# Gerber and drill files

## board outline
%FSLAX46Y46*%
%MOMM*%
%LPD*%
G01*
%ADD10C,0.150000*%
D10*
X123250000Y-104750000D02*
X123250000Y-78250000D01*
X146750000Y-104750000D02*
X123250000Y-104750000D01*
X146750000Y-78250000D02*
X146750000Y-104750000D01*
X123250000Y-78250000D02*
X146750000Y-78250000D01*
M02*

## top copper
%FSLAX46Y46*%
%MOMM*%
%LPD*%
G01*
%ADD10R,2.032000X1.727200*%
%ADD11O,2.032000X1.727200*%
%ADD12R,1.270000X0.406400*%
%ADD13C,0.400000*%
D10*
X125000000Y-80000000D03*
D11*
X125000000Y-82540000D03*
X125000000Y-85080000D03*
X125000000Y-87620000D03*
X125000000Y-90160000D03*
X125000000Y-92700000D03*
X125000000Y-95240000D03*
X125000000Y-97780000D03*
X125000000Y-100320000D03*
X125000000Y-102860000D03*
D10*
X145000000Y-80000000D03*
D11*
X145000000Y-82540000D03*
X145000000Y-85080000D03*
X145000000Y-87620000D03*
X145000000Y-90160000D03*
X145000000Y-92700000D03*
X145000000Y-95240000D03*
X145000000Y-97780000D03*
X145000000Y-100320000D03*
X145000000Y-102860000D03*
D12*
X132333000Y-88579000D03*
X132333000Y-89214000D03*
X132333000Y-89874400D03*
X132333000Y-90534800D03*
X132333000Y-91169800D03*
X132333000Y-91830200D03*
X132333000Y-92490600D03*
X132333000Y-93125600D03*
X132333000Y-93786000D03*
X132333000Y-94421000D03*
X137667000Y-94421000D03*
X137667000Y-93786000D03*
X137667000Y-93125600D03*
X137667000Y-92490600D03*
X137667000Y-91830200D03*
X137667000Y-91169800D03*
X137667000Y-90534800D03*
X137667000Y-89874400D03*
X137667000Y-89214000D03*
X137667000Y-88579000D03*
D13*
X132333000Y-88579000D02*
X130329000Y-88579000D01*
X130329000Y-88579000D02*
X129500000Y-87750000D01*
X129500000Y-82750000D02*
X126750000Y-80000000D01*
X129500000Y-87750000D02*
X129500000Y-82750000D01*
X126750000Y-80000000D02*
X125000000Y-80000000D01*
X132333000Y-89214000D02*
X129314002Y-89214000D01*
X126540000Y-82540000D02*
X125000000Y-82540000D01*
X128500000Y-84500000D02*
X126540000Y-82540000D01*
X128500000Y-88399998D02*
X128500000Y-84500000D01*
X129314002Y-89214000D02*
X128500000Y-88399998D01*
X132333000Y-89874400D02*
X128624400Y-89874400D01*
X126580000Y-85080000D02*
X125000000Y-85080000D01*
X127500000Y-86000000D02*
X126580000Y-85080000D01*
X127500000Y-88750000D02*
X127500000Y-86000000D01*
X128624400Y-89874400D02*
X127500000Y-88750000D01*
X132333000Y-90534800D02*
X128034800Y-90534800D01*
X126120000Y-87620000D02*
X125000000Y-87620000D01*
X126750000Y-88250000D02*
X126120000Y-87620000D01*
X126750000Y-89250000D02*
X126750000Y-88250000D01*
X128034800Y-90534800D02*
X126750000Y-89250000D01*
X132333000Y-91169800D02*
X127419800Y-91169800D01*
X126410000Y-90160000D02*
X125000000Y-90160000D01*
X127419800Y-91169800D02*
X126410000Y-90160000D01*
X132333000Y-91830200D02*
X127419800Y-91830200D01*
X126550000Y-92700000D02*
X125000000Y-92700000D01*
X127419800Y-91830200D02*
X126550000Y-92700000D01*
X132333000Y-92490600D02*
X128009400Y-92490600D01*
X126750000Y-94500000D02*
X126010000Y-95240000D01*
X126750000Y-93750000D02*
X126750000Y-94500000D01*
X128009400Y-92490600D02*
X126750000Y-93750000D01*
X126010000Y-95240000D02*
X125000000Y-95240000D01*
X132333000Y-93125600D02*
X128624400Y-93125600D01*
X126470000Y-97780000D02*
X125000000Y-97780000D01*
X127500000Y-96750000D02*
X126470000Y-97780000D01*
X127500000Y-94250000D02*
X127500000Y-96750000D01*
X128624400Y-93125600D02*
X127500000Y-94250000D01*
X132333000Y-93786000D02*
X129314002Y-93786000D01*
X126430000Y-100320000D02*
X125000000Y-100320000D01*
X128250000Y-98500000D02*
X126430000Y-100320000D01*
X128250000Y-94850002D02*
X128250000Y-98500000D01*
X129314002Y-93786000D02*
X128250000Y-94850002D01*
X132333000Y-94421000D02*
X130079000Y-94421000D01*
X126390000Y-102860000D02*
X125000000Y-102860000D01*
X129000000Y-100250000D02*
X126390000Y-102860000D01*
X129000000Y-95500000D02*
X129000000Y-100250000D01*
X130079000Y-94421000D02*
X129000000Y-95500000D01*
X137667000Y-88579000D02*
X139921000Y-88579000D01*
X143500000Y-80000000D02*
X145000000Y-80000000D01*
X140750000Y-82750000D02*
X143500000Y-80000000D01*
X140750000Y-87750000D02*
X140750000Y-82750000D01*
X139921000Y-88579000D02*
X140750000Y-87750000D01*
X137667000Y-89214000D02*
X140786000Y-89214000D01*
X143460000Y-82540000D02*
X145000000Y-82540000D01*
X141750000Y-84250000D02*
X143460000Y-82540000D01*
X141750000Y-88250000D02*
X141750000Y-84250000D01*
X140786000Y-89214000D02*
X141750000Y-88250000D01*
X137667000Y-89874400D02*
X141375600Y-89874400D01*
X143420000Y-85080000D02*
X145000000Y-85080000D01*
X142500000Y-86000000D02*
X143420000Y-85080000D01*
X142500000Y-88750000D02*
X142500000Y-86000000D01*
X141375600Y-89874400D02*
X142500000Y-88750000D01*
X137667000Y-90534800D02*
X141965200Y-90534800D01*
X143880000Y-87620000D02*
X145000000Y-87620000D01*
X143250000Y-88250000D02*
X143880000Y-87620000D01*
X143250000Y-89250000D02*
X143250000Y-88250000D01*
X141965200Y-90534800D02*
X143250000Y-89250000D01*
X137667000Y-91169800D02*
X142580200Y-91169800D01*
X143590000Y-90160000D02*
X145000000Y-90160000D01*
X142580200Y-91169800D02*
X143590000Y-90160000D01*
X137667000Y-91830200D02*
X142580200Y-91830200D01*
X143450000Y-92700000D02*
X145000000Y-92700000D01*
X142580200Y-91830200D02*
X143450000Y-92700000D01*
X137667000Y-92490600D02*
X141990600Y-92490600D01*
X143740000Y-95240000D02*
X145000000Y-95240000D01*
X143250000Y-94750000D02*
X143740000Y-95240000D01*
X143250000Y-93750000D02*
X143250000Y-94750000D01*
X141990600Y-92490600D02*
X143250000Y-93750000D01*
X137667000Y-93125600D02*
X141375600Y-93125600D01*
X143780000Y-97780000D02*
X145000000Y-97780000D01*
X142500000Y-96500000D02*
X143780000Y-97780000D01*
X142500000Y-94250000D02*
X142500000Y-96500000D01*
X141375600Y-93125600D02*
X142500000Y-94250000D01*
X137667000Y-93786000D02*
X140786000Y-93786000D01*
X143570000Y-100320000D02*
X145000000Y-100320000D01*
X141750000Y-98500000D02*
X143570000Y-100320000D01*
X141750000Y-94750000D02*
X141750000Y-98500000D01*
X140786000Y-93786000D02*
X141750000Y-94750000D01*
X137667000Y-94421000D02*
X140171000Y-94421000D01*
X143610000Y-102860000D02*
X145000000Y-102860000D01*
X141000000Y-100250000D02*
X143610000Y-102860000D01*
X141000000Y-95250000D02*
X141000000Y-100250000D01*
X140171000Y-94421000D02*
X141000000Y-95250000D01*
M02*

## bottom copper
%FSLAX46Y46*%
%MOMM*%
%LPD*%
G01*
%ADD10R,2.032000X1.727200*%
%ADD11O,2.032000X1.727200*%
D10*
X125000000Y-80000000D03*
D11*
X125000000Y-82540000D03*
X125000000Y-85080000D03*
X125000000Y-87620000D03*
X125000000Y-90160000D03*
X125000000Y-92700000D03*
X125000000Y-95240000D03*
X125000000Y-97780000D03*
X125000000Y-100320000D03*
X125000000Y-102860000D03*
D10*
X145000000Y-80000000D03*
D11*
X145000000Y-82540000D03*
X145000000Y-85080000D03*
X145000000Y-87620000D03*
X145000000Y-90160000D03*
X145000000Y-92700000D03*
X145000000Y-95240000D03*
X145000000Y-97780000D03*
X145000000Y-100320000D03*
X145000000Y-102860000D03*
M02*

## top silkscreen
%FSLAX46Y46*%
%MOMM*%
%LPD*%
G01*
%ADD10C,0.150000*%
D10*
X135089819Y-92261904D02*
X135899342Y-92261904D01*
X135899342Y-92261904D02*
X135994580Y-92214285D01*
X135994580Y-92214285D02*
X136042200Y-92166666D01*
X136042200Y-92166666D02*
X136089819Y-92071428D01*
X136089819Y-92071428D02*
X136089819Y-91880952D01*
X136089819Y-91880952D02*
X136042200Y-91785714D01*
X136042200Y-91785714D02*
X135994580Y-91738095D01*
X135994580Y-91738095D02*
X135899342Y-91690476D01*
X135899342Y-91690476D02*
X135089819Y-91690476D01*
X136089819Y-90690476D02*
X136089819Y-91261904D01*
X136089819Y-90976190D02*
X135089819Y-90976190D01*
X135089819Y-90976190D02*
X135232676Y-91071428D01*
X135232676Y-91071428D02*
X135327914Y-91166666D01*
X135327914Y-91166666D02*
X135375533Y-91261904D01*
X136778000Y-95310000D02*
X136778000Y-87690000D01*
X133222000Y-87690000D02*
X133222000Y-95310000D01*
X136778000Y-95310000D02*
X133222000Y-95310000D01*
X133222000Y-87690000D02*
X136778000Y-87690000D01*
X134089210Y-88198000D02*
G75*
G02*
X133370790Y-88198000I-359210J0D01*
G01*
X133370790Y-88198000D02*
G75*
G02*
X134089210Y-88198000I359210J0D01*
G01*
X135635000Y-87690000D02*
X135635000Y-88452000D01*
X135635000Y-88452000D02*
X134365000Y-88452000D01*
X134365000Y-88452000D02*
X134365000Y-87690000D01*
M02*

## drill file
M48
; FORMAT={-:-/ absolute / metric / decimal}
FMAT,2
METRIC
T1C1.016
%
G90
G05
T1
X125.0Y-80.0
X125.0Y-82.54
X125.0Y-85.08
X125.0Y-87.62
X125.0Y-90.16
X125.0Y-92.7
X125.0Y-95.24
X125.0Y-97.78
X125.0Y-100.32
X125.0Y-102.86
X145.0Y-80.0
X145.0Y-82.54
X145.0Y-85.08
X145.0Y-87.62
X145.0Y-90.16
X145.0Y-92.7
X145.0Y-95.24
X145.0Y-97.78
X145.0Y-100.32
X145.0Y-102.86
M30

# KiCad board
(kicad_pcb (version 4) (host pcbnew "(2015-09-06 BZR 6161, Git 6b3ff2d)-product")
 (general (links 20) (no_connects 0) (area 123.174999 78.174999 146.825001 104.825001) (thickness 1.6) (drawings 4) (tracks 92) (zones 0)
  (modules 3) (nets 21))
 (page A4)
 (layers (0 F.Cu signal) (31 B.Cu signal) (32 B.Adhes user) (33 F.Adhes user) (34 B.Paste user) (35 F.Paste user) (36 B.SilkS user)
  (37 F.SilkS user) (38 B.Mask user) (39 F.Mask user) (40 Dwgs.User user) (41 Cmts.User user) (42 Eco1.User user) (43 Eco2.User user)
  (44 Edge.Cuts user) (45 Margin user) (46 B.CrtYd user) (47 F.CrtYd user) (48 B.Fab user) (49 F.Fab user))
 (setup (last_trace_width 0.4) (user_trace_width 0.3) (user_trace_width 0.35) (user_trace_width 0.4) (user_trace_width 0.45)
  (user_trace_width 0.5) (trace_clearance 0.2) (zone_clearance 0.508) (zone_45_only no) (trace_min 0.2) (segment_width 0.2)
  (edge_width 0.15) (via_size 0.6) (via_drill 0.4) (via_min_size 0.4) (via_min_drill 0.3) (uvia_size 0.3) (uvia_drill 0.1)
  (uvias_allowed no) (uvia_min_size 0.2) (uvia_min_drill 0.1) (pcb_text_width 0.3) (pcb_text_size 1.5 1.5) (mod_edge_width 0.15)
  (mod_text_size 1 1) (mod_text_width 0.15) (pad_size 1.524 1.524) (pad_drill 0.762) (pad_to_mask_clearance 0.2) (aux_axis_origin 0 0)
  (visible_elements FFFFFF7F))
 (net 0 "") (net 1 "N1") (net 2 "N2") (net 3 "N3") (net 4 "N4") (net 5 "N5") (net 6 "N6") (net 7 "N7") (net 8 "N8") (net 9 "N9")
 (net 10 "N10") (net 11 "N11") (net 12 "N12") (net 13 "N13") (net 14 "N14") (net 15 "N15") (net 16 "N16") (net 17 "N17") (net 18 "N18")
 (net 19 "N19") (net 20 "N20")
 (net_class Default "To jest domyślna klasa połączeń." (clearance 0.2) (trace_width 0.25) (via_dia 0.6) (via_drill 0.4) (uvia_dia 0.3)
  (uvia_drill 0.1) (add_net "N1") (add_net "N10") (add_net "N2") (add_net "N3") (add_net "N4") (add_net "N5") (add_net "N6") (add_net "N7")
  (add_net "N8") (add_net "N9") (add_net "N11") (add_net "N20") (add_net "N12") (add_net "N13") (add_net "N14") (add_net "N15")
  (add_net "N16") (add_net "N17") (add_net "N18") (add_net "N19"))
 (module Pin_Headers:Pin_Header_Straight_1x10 (layer B.Cu) (at 125 80 180)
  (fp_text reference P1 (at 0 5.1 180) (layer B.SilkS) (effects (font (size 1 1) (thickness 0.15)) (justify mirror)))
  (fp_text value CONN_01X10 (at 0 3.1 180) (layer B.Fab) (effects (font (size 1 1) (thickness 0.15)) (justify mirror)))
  (pad 1 thru_hole rect (at 0 0 180) (size 2.032 1.7272) (drill 1.016) (layers *.Cu *.Mask B.SilkS) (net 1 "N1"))
  (pad 2 thru_hole oval (at 0 -2.54 180) (size 2.032 1.7272) (drill 1.016) (layers *.Cu *.Mask B.SilkS) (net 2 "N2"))
  (pad 3 thru_hole oval (at 0 -5.08 180) (size 2.032 1.7272) (drill 1.016) (layers *.Cu *.Mask B.SilkS) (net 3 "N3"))
  (pad 4 thru_hole oval (at 0 -7.62 180) (size 2.032 1.7272) (drill 1.016) (layers *.Cu *.Mask B.SilkS) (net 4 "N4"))
  (pad 5 thru_hole oval (at 0 -10.16 180) (size 2.032 1.7272) (drill 1.016) (layers *.Cu *.Mask B.SilkS) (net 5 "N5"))
  (pad 6 thru_hole oval (at 0 -12.7 180) (size 2.032 1.7272) (drill 1.016) (layers *.Cu *.Mask B.SilkS) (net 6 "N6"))
  (pad 7 thru_hole oval (at 0 -15.24 180) (size 2.032 1.7272) (drill 1.016) (layers *.Cu *.Mask B.SilkS) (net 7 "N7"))
  (pad 8 thru_hole oval (at 0 -17.78 180) (size 2.032 1.7272) (drill 1.016) (layers *.Cu *.Mask B.SilkS) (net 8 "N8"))
  (pad 9 thru_hole oval (at 0 -20.32 180) (size 2.032 1.7272) (drill 1.016) (layers *.Cu *.Mask B.SilkS) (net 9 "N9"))
  (pad 10 thru_hole oval (at 0 -22.86 180) (size 2.032 1.7272) (drill 1.016) (layers *.Cu *.Mask B.SilkS) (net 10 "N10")))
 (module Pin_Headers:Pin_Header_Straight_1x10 (layer B.Cu) (at 145 80 180)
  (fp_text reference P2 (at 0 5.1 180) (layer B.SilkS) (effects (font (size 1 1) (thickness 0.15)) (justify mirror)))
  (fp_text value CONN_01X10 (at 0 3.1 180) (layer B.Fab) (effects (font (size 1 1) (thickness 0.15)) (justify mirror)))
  (pad 1 thru_hole rect (at 0 0 180) (size 2.032 1.7272) (drill 1.016) (layers *.Cu *.Mask B.SilkS) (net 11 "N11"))
  (pad 2 thru_hole oval (at 0 -2.54 180) (size 2.032 1.7272) (drill 1.016) (layers *.Cu *.Mask B.SilkS) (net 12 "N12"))
  (pad 3 thru_hole oval (at 0 -5.08 180) (size 2.032 1.7272) (drill 1.016) (layers *.Cu *.Mask B.SilkS) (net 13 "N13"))
  (pad 4 thru_hole oval (at 0 -7.62 180) (size 2.032 1.7272) (drill 1.016) (layers *.Cu *.Mask B.SilkS) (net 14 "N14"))
  (pad 5 thru_hole oval (at 0 -10.16 180) (size 2.032 1.7272) (drill 1.016) (layers *.Cu *.Mask B.SilkS) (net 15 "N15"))
  (pad 6 thru_hole oval (at 0 -12.7 180) (size 2.032 1.7272) (drill 1.016) (layers *.Cu *.Mask B.SilkS) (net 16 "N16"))
  (pad 7 thru_hole oval (at 0 -15.24 180) (size 2.032 1.7272) (drill 1.016) (layers *.Cu *.Mask B.SilkS) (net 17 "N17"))
  (pad 8 thru_hole oval (at 0 -17.78 180) (size 2.032 1.7272) (drill 1.016) (layers *.Cu *.Mask B.SilkS) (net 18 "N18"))
  (pad 9 thru_hole oval (at 0 -20.32 180) (size 2.032 1.7272) (drill 1.016) (layers *.Cu *.Mask B.SilkS) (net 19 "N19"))
  (pad 10 thru_hole oval (at 0 -22.86 180) (size 2.032 1.7272) (drill 1.016) (layers *.Cu *.Mask B.SilkS) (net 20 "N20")))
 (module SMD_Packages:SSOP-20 (layer F.Cu) (at 135 91.5 270)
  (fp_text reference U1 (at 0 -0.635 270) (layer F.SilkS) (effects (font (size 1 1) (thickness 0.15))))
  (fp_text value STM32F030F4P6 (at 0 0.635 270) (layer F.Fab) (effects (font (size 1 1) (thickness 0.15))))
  (fp_line (start 3.81 -1.778) (end -3.81 -1.778) (layer F.SilkS) (width 0.15))
  (fp_line (start -3.81 1.778) (end 3.81 1.778) (layer F.SilkS) (width 0.15))
  (fp_line (start 3.81 -1.778) (end 3.81 1.778) (layer F.SilkS) (width 0.15))
  (fp_line (start -3.81 1.778) (end -3.81 -1.778) (layer F.SilkS) (width 0.15))
  (fp_circle (center -3.302 1.27) (end -3.556 1.016) (layer F.SilkS) (width 0.15))
  (fp_line (start -3.81 -0.635) (end -3.048 -0.635) (layer F.SilkS) (width 0.15))
  (fp_line (start -3.048 -0.635) (end -3.048 0.635) (layer F.SilkS) (width 0.15))
  (fp_line (start -3.048 0.635) (end -3.81 0.635) (layer F.SilkS) (width 0.15))
  (pad 1 smd rect (at -2.921 2.667 270) (size 0.4064 1.27) (layers F.Cu F.Paste F.Mask) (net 1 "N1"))
  (pad 2 smd rect (at -2.286 2.667 270) (size 0.4064 1.27) (layers F.Cu F.Paste F.Mask) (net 2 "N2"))
  (pad 3 smd rect (at -1.6256 2.667 270) (size 0.4064 1.27) (layers F.Cu F.Paste F.Mask) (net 3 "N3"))
  (pad 4 smd rect (at -0.9652 2.667 270) (size 0.4064 1.27) (layers F.Cu F.Paste F.Mask) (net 4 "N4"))
  (pad 5 smd rect (at -0.3302 2.667 270) (size 0.4064 1.27) (layers F.Cu F.Paste F.Mask) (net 5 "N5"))
  (pad 6 smd rect (at 0.3302 2.667 270) (size 0.4064 1.27) (layers F.Cu F.Paste F.Mask) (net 6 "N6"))
  (pad 7 smd rect (at 0.9906 2.667 270) (size 0.4064 1.27) (layers F.Cu F.Paste F.Mask) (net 7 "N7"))
  (pad 8 smd rect (at 1.6256 2.667 270) (size 0.4064 1.27) (layers F.Cu F.Paste F.Mask) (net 8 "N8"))
  (pad 9 smd rect (at 2.286 2.667 270) (size 0.4064 1.27) (layers F.Cu F.Paste F.Mask) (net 9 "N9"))
  (pad 10 smd rect (at 2.921 2.667 270) (size 0.4064 1.27) (layers F.Cu F.Paste F.Mask) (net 10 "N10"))
  (pad 11 smd rect (at 2.921 -2.667 270) (size 0.4064 1.27) (layers F.Cu F.Paste F.Mask) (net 20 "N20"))
  (pad 12 smd rect (at 2.286 -2.667 270) (size 0.4064 1.27) (layers F.Cu F.Paste F.Mask) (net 19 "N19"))
  (pad 13 smd rect (at 1.6256 -2.667 270) (size 0.4064 1.27) (layers F.Cu F.Paste F.Mask) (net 18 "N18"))
  (pad 14 smd rect (at 0.9906 -2.667 270) (size 0.4064 1.27) (layers F.Cu F.Paste F.Mask) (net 17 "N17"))
  (pad 15 smd rect (at 0.3302 -2.667 270) (size 0.4064 1.27) (layers F.Cu F.Paste F.Mask) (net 16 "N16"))
  (pad 16 smd rect (at -0.3302 -2.667 270) (size 0.4064 1.27) (layers F.Cu F.Paste F.Mask) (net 15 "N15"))
  (pad 17 smd rect (at -0.9652 -2.667 270) (size 0.4064 1.27) (layers F.Cu F.Paste F.Mask) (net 14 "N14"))
  (pad 18 smd rect (at -1.6256 -2.667 270) (size 0.4064 1.27) (layers F.Cu F.Paste F.Mask) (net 13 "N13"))
  (pad 19 smd rect (at -2.286 -2.667 270) (size 0.4064 1.27) (layers F.Cu F.Paste F.Mask) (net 12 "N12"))
  (pad 20 smd rect (at -2.921 -2.667 270) (size 0.4064 1.27) (layers F.Cu F.Paste F.Mask) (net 11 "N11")))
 (gr_line (start 123.25 104.75) (end 123.25 78.25) (angle 90) (layer Edge.Cuts) (width 0.15))
 (gr_line (start 146.75 104.75) (end 123.25 104.75) (angle 90) (layer Edge.Cuts) (width 0.15))
 (gr_line (start 146.75 78.25) (end 146.75 104.75) (angle 90) (layer Edge.Cuts) (width 0.15))
 (gr_line (start 123.25 78.25) (end 146.75 78.25) (angle 90) (layer Edge.Cuts) (width 0.15))
 (segment (start 132.333 88.579) (end 130.329 88.579) (width 0.4) (layer F.Cu) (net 1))
 (segment (start 130.329 88.579) (end 129.5 87.75) (width 0.4) (layer F.Cu) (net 1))
 (segment (start 129.5 82.75) (end 126.75 80) (width 0.4) (layer F.Cu) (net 1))
 (segment (start 129.5 87.75) (end 129.5 82.75) (width 0.4) (layer F.Cu) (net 1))
 (segment (start 126.75 80) (end 125 80) (width 0.4) (layer F.Cu) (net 1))
 (segment (start 132.333 89.214) (end 129.314002 89.214) (width 0.4) (layer F.Cu) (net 2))
 (segment (start 126.54 82.54) (end 125 82.54) (width 0.4) (layer F.Cu) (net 2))
 (segment (start 128.5 84.5) (end 126.54 82.54) (width 0.4) (layer F.Cu) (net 2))
 (segment (start 128.5 88.399998) (end 128.5 84.5) (width 0.4) (layer F.Cu) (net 2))
 (segment (start 129.314002 89.214) (end 128.5 88.399998) (width 0.4) (layer F.Cu) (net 2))
 (segment (start 132.333 89.8744) (end 128.6244 89.8744) (width 0.4) (layer F.Cu) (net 3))
 (segment (start 126.58 85.08) (end 125 85.08) (width 0.4) (layer F.Cu) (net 3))
 (segment (start 127.5 86) (end 126.58 85.08) (width 0.4) (layer F.Cu) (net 3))
 (segment (start 127.5 88.75) (end 127.5 86) (width 0.4) (layer F.Cu) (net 3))
 (segment (start 128.6244 89.8744) (end 127.5 88.75) (width 0.4) (layer F.Cu) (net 3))
 (segment (start 132.333 90.5348) (end 128.0348 90.5348) (width 0.4) (layer F.Cu) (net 4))
 (segment (start 126.12 87.62) (end 125 87.62) (width 0.4) (layer F.Cu) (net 4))
 (segment (start 126.75 88.25) (end 126.12 87.62) (width 0.4) (layer F.Cu) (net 4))
 (segment (start 126.75 89.25) (end 126.75 88.25) (width 0.4) (layer F.Cu) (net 4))
 (segment (start 128.0348 90.5348) (end 126.75 89.25) (width 0.4) (layer F.Cu) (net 4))
 (segment (start 132.333 91.1698) (end 127.4198 91.1698) (width 0.4) (layer F.Cu) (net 5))
 (segment (start 126.41 90.16) (end 125 90.16) (width 0.4) (layer F.Cu) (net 5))
 (segment (start 127.4198 91.1698) (end 126.41 90.16) (width 0.4) (layer F.Cu) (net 5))
 (segment (start 132.333 91.8302) (end 127.4198 91.8302) (width 0.4) (layer F.Cu) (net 6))
 (segment (start 126.55 92.7) (end 125 92.7) (width 0.4) (layer F.Cu) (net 6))
 (segment (start 127.4198 91.8302) (end 126.55 92.7) (width 0.4) (layer F.Cu) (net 6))
 (segment (start 132.333 92.4906) (end 128.0094 92.4906) (width 0.4) (layer F.Cu) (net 7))
 (segment (start 126.75 94.5) (end 126.01 95.24) (width 0.4) (layer F.Cu) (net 7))
 (segment (start 126.75 93.75) (end 126.75 94.5) (width 0.4) (layer F.Cu) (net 7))
 (segment (start 128.0094 92.4906) (end 126.75 93.75) (width 0.4) (layer F.Cu) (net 7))
 (segment (start 126.01 95.24) (end 125 95.24) (width 0.4) (layer F.Cu) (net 7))
 (segment (start 132.333 93.1256) (end 128.6244 93.1256) (width 0.4) (layer F.Cu) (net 8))
 (segment (start 126.47 97.78) (end 125 97.78) (width 0.4) (layer F.Cu) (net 8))
 (segment (start 127.5 96.75) (end 126.47 97.78) (width 0.4) (layer F.Cu) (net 8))
 (segment (start 127.5 94.25) (end 127.5 96.75) (width 0.4) (layer F.Cu) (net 8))
 (segment (start 128.6244 93.1256) (end 127.5 94.25) (width 0.4) (layer F.Cu) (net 8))
 (segment (start 132.333 93.786) (end 129.314002 93.786) (width 0.4) (layer F.Cu) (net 9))
 (segment (start 126.43 100.32) (end 125 100.32) (width 0.4) (layer F.Cu) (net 9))
 (segment (start 128.25 98.5) (end 126.43 100.32) (width 0.4) (layer F.Cu) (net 9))
 (segment (start 128.25 94.850002) (end 128.25 98.5) (width 0.4) (layer F.Cu) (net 9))
 (segment (start 129.314002 93.786) (end 128.25 94.850002) (width 0.4) (layer F.Cu) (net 9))
 (segment (start 132.333 94.421) (end 130.079 94.421) (width 0.4) (layer F.Cu) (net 10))
 (segment (start 126.39 102.86) (end 125 102.86) (width 0.4) (layer F.Cu) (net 10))
 (segment (start 129 100.25) (end 126.39 102.86) (width 0.4) (layer F.Cu) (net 10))
 (segment (start 129 95.5) (end 129 100.25) (width 0.4) (layer F.Cu) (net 10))
 (segment (start 130.079 94.421) (end 129 95.5) (width 0.4) (layer F.Cu) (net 10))
 (segment (start 137.667 88.579) (end 139.921 88.579) (width 0.4) (layer F.Cu) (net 11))
 (segment (start 143.5 80) (end 145 80) (width 0.4) (layer F.Cu) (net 11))
 (segment (start 140.75 82.75) (end 143.5 80) (width 0.4) (layer F.Cu) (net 11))
 (segment (start 140.75 87.75) (end 140.75 82.75) (width 0.4) (layer F.Cu) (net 11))
 (segment (start 139.921 88.579) (end 140.75 87.75) (width 0.4) (layer F.Cu) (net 11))
 (segment (start 137.667 89.214) (end 140.786 89.214) (width 0.4) (layer F.Cu) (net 12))
 (segment (start 143.46 82.54) (end 145 82.54) (width 0.4) (layer F.Cu) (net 12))
 (segment (start 141.75 84.25) (end 143.46 82.54) (width 0.4) (layer F.Cu) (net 12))
 (segment (start 141.75 88.25) (end 141.75 84.25) (width 0.4) (layer F.Cu) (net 12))
 (segment (start 140.786 89.214) (end 141.75 88.25) (width 0.4) (layer F.Cu) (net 12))
 (segment (start 137.667 89.8744) (end 141.3756 89.8744) (width 0.4) (layer F.Cu) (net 13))
 (segment (start 143.42 85.08) (end 145 85.08) (width 0.4) (layer F.Cu) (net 13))
 (segment (start 142.5 86) (end 143.42 85.08) (width 0.4) (layer F.Cu) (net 13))
 (segment (start 142.5 88.75) (end 142.5 86) (width 0.4) (layer F.Cu) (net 13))
 (segment (start 141.3756 89.8744) (end 142.5 88.75) (width 0.4) (layer F.Cu) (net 13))
 (segment (start 137.667 90.5348) (end 141.9652 90.5348) (width 0.4) (layer F.Cu) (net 14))
 (segment (start 143.88 87.62) (end 145 87.62) (width 0.4) (layer F.Cu) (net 14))
 (segment (start 143.25 88.25) (end 143.88 87.62) (width 0.4) (layer F.Cu) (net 14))
 (segment (start 143.25 89.25) (end 143.25 88.25) (width 0.4) (layer F.Cu) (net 14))
 (segment (start 141.9652 90.5348) (end 143.25 89.25) (width 0.4) (layer F.Cu) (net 14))
 (segment (start 137.667 91.1698) (end 142.5802 91.1698) (width 0.4) (layer F.Cu) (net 15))
 (segment (start 143.59 90.16) (end 145 90.16) (width 0.4) (layer F.Cu) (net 15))
 (segment (start 142.5802 91.1698) (end 143.59 90.16) (width 0.4) (layer F.Cu) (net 15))
 (segment (start 137.667 91.8302) (end 142.5802 91.8302) (width 0.4) (layer F.Cu) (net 16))
 (segment (start 143.45 92.7) (end 145 92.7) (width 0.4) (layer F.Cu) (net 16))
 (segment (start 142.5802 91.8302) (end 143.45 92.7) (width 0.4) (layer F.Cu) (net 16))
 (segment (start 137.667 92.4906) (end 141.9906 92.4906) (width 0.4) (layer F.Cu) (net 17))
 (segment (start 143.74 95.24) (end 145 95.24) (width 0.4) (layer F.Cu) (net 17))
 (segment (start 143.25 94.75) (end 143.74 95.24) (width 0.4) (layer F.Cu) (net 17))
 (segment (start 143.25 93.75) (end 143.25 94.75) (width 0.4) (layer F.Cu) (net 17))
 (segment (start 141.9906 92.4906) (end 143.25 93.75) (width 0.4) (layer F.Cu) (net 17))
 (segment (start 137.667 93.1256) (end 141.3756 93.1256) (width 0.4) (layer F.Cu) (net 18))
 (segment (start 143.78 97.78) (end 145 97.78) (width 0.4) (layer F.Cu) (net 18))
 (segment (start 142.5 96.5) (end 143.78 97.78) (width 0.4) (layer F.Cu) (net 18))
 (segment (start 142.5 94.25) (end 142.5 96.5) (width 0.4) (layer F.Cu) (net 18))
 (segment (start 141.3756 93.1256) (end 142.5 94.25) (width 0.4) (layer F.Cu) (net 18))
 (segment (start 137.667 93.786) (end 140.786 93.786) (width 0.4) (layer F.Cu) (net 19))
 (segment (start 143.57 100.32) (end 145 100.32) (width 0.4) (layer F.Cu) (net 19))
 (segment (start 141.75 98.5) (end 143.57 100.32) (width 0.4) (layer F.Cu) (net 19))
 (segment (start 141.75 94.75) (end 141.75 98.5) (width 0.4) (layer F.Cu) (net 19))
 (segment (start 140.786 93.786) (end 141.75 94.75) (width 0.4) (layer F.Cu) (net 19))
 (segment (start 137.667 94.421) (end 140.171 94.421) (width 0.4) (layer F.Cu) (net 20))
 (segment (start 143.61 102.86) (end 145 102.86) (width 0.4) (layer F.Cu) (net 20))
 (segment (start 141 100.25) (end 143.61 102.86) (width 0.4) (layer F.Cu) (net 20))
 (segment (start 141 95.25) (end 141 100.25) (width 0.4) (layer F.Cu) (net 20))
 (segment (start 140.171 94.421) (end 141 95.25) (width 0.4) (layer F.Cu) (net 20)))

